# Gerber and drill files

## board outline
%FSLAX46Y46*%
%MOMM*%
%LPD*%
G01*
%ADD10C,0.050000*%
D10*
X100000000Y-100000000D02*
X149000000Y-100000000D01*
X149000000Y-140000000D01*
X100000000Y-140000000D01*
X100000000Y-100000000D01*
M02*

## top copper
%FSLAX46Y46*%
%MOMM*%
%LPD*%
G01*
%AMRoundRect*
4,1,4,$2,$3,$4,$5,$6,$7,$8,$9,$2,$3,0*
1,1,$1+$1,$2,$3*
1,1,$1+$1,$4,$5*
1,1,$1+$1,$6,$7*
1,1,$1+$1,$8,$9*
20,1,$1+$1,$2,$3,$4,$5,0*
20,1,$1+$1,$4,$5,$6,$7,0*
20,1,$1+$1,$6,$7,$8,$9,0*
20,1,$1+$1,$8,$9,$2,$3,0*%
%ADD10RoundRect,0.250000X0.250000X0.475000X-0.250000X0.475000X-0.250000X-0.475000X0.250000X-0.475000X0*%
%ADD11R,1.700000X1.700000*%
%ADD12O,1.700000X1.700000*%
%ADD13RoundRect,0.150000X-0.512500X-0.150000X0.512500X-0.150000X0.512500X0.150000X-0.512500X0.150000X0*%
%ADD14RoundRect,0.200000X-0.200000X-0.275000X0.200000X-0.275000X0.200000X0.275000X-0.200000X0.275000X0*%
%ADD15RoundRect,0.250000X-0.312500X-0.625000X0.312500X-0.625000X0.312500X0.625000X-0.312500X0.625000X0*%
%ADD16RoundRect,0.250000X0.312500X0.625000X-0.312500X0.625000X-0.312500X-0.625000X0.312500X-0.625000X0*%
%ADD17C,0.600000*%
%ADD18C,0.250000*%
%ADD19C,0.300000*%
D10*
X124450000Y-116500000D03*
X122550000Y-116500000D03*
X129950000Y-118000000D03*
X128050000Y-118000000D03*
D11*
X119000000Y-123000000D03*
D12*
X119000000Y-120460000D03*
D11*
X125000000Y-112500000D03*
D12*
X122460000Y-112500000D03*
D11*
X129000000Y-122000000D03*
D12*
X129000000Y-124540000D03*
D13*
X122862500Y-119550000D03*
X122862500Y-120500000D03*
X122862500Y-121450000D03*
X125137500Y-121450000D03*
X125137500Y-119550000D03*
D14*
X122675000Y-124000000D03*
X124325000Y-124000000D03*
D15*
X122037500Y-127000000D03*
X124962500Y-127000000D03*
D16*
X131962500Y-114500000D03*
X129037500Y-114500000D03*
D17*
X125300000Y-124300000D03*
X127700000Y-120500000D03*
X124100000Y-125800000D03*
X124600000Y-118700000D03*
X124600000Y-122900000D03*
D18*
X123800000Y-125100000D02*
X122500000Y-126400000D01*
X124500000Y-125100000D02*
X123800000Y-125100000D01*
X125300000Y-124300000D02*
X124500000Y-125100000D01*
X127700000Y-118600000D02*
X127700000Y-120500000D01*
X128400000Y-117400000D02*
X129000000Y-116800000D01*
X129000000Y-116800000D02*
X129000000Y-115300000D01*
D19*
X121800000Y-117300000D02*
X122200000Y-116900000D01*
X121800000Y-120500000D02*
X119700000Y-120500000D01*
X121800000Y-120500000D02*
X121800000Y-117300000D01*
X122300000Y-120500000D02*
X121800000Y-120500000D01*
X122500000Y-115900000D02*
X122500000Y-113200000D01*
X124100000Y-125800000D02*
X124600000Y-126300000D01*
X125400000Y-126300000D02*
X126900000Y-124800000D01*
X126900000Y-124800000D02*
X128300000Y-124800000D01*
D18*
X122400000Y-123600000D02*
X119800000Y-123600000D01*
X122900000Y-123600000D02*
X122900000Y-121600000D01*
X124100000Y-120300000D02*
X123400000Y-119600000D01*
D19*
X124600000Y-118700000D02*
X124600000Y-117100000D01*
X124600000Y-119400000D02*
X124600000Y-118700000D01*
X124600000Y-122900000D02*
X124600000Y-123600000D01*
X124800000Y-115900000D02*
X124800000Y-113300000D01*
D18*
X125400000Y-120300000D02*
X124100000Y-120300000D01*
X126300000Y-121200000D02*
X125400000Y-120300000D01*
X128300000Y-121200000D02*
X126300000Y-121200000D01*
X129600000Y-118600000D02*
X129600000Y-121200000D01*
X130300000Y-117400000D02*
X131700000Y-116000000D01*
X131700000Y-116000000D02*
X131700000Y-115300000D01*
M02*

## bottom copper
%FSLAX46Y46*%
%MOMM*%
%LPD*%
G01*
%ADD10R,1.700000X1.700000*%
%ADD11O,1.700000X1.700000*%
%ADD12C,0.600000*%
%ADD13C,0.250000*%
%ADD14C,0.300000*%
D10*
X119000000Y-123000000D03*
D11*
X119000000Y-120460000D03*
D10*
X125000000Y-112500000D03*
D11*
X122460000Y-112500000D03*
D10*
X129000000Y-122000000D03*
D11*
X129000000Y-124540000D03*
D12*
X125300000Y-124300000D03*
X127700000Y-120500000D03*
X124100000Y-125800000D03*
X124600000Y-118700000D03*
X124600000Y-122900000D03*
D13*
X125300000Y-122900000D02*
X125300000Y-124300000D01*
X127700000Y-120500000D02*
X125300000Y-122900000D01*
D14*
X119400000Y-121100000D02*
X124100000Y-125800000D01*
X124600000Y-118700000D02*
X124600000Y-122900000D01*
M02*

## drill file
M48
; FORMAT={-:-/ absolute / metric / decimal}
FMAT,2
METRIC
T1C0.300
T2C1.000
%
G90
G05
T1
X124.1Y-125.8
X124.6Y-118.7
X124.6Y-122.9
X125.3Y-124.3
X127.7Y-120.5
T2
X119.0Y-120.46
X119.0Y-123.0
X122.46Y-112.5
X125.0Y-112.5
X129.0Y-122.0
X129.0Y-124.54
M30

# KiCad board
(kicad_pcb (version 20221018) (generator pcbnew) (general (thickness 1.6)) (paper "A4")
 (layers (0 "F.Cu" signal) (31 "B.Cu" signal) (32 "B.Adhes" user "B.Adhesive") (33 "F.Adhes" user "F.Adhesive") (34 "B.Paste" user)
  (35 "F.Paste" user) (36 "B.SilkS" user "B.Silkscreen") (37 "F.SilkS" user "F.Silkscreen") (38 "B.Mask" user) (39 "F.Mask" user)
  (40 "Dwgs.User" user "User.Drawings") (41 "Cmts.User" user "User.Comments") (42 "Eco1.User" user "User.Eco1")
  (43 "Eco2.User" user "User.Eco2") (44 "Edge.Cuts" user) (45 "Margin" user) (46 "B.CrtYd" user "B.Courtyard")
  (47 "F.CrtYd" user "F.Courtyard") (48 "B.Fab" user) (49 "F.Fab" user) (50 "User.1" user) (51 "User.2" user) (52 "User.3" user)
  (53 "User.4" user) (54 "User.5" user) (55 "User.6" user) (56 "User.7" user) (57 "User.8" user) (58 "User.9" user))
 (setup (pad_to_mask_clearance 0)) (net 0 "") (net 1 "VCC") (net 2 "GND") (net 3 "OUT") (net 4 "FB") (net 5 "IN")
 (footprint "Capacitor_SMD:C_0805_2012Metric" (layer "F.Cu") (at 123.5 116.5 180)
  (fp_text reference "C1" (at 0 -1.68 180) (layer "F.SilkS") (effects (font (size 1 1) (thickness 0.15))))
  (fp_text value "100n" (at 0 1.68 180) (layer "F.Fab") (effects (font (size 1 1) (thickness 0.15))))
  (pad "1" smd roundrect (at -0.95 0 180) (size 1 1.45) (layers "F.Cu" "F.Paste" "F.Mask") (roundrect_rratio 0.25) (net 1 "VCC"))
  (pad "2" smd roundrect (at 0.95 0 180) (size 1 1.45) (layers "F.Cu" "F.Paste" "F.Mask") (roundrect_rratio 0.25) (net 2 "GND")))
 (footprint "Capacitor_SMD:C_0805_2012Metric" (layer "F.Cu") (at 129 118 180)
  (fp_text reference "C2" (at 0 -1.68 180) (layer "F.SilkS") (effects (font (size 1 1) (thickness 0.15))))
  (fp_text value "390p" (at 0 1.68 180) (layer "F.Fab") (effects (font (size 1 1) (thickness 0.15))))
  (pad "1" smd roundrect (at -0.95 0 180) (size 1 1.45) (layers "F.Cu" "F.Paste" "F.Mask") (roundrect_rratio 0.25) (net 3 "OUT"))
  (pad "2" smd roundrect (at 0.95 0 180) (size 1 1.45) (layers "F.Cu" "F.Paste" "F.Mask") (roundrect_rratio 0.25) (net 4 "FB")))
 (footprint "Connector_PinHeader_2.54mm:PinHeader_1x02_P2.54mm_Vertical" (layer "F.Cu") (at 119 123 180)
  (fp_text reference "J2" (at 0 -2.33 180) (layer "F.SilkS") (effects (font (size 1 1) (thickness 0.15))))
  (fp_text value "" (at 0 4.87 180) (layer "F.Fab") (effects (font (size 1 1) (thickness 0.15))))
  (pad "1" thru_hole rect (at 0 0 180) (size 1.7 1.7) (drill 1) (layers "*.Cu" "*.Mask") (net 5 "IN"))
  (pad "2" thru_hole oval (at 0 2.54 180) (size 1.7 1.7) (drill 1) (layers "*.Cu" "*.Mask") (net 2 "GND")))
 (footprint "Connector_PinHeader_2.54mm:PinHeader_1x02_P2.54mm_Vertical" (layer "F.Cu") (at 125 112.5 -90)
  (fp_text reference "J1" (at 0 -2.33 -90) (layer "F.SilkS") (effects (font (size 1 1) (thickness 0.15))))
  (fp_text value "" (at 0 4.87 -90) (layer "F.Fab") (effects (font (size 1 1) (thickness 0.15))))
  (pad "1" thru_hole rect (at 0 0 270) (size 1.7 1.7) (drill 1) (layers "*.Cu" "*.Mask") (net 1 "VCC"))
  (pad "2" thru_hole oval (at 0 2.54 270) (size 1.7 1.7) (drill 1) (layers "*.Cu" "*.Mask") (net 2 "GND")))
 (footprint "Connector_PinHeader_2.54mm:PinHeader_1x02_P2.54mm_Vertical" (layer "F.Cu") (at 129 122)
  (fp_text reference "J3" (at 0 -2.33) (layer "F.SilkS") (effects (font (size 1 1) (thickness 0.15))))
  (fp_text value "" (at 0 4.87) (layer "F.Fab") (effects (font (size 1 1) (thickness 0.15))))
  (pad "1" thru_hole rect (at 0 0) (size 1.7 1.7) (drill 1) (layers "*.Cu" "*.Mask") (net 3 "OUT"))
  (pad "2" thru_hole oval (at 0 2.54) (size 1.7 1.7) (drill 1) (layers "*.Cu" "*.Mask") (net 2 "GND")))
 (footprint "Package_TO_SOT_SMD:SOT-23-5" (layer "F.Cu") (at 124 120.5)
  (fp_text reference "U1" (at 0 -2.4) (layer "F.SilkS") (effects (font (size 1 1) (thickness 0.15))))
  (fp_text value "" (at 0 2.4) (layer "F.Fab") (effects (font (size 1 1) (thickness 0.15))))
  (pad "1" smd roundrect (at -1.1375 -0.95) (size 1.325 0.6) (layers "F.Cu" "F.Paste" "F.Mask") (roundrect_rratio 0.25) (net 3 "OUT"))
  (pad "2" smd roundrect (at -1.1375 0) (size 1.325 0.6) (layers "F.Cu" "F.Paste" "F.Mask") (roundrect_rratio 0.25) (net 2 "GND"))
  (pad "3" smd roundrect (at -1.1375 0.95) (size 1.325 0.6) (layers "F.Cu" "F.Paste" "F.Mask") (roundrect_rratio 0.25) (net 5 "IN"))
  (pad "4" smd roundrect (at 1.1375 0.95) (size 1.325 0.6) (layers "F.Cu" "F.Paste" "F.Mask") (roundrect_rratio 0.25))
  (pad "5" smd roundrect (at 1.1375 -0.95) (size 1.325 0.6) (layers "F.Cu" "F.Paste" "F.Mask") (roundrect_rratio 0.25) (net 1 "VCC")))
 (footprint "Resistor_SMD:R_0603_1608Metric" (layer "F.Cu") (at 123.5 124)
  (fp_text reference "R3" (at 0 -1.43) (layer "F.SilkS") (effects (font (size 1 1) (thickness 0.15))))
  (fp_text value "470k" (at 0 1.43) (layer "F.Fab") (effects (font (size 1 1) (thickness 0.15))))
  (pad "1" smd roundrect (at -0.825 0) (size 0.8 0.95) (layers "F.Cu" "F.Paste" "F.Mask") (roundrect_rratio 0.25) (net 5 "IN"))
  (pad "2" smd roundrect (at 0.825 0) (size 0.8 0.95) (layers "F.Cu" "F.Paste" "F.Mask") (roundrect_rratio 0.25) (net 1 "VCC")))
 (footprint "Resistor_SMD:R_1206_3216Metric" (layer "F.Cu") (at 123.5 127)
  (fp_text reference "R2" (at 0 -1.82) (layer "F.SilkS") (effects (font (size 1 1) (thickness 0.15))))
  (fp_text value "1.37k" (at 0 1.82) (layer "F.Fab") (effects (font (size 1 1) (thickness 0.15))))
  (pad "1" smd roundrect (at -1.4625 0) (size 1.125 1.75) (layers "F.Cu" "F.Paste" "F.Mask") (roundrect_rratio 0.222222) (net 4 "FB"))
  (pad "2" smd roundrect (at 1.4625 0) (size 1.125 1.75) (layers "F.Cu" "F.Paste" "F.Mask") (roundrect_rratio 0.222222) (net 2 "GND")))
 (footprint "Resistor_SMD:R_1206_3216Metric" (layer "F.Cu") (at 130.5 114.5 180)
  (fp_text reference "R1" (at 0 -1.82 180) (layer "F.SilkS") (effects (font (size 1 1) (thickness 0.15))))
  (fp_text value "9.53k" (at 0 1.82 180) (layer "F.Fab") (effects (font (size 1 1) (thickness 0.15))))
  (pad "1" smd roundrect (at -1.4625 0 180) (size 1.125 1.75) (layers "F.Cu" "F.Paste" "F.Mask") (roundrect_rratio 0.222222) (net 3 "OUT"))
  (pad "2" smd roundrect (at 1.4625 0 180) (size 1.125 1.75) (layers "F.Cu" "F.Paste" "F.Mask") (roundrect_rratio 0.222222) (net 4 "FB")))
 (gr_rect (start 100 100) (end 149 140) (stroke (width 0.05) (type default)) (fill none) (layer "Edge.Cuts"))
 (segment (start 123.8 125.1) (end 122.5 126.4) (width 0.25) (layer "F.Cu") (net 4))
 (segment (start 124.5 125.1) (end 123.8 125.1) (width 0.25) (layer "F.Cu") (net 4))
 (segment (start 125.3 124.3) (end 124.5 125.1) (width 0.25) (layer "F.Cu") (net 4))
 (segment (start 127.7 118.6) (end 127.7 120.5) (width 0.25) (layer "F.Cu") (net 4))
 (segment (start 128.4 117.4) (end 129 116.8) (width 0.25) (layer "F.Cu") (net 4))
 (segment (start 129 116.8) (end 129 115.3) (width 0.25) (layer "F.Cu") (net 4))
 (via (at 125.3 124.3) (size 0.6) (drill 0.3) (layers "F.Cu" "B.Cu") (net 4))
 (via (at 127.7 120.5) (size 0.6) (drill 0.3) (layers "F.Cu" "B.Cu") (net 4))
 (segment (start 121.8 117.3) (end 122.2 116.9) (width 0.3) (layer "F.Cu") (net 2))
 (segment (start 121.8 120.5) (end 119.7 120.5) (width 0.3) (layer "F.Cu") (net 2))
 (segment (start 121.8 120.5) (end 121.8 117.3) (width 0.3) (layer "F.Cu") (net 2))
 (segment (start 122.3 120.5) (end 121.8 120.5) (width 0.3) (layer "F.Cu") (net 2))
 (segment (start 122.5 115.9) (end 122.5 113.2) (width 0.3) (layer "F.Cu") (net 2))
 (segment (start 124.1 125.8) (end 124.6 126.3) (width 0.3) (layer "F.Cu") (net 2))
 (segment (start 125.3 122.9) (end 125.3 124.3) (width 0.25) (layer "B.Cu") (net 4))
 (segment (start 125.4 126.3) (end 126.9 124.8) (width 0.3) (layer "F.Cu") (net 2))
 (segment (start 126.9 124.8) (end 128.3 124.8) (width 0.3) (layer "F.Cu") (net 2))
 (segment (start 127.7 120.5) (end 125.3 122.9) (width 0.25) (layer "B.Cu") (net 4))
 (via (at 124.1 125.8) (size 0.6) (drill 0.3) (layers "F.Cu" "B.Cu") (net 2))
 (segment (start 119.4 121.1) (end 124.1 125.8) (width 0.3) (layer "B.Cu") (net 2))
 (segment (start 122.4 123.6) (end 119.8 123.6) (width 0.25) (layer "F.Cu") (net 5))
 (segment (start 122.9 123.6) (end 122.9 121.6) (width 0.25) (layer "F.Cu") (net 5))
 (segment (start 124.1 120.3) (end 123.4 119.6) (width 0.25) (layer "F.Cu") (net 3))
 (segment (start 124.6 118.7) (end 124.6 117.1) (width 0.3) (layer "F.Cu") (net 1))
 (segment (start 124.6 119.4) (end 124.6 118.7) (width 0.3) (layer "F.Cu") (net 1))
 (segment (start 124.6 122.9) (end 124.6 123.6) (width 0.3) (layer "F.Cu") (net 1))
 (segment (start 124.8 115.9) (end 124.8 113.3) (width 0.3) (layer "F.Cu") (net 1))
 (segment (start 125.4 120.3) (end 124.1 120.3) (width 0.25) (layer "F.Cu") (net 3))
 (segment (start 126.3 121.2) (end 125.4 120.3) (width 0.25) (layer "F.Cu") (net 3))
 (segment (start 128.3 121.2) (end 126.3 121.2) (width 0.25) (layer "F.Cu") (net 3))
 (segment (start 129.6 118.6) (end 129.6 121.2) (width 0.25) (layer "F.Cu") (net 3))
 (segment (start 130.3 117.4) (end 131.7 116) (width 0.25) (layer "F.Cu") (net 3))
 (segment (start 131.7 116) (end 131.7 115.3) (width 0.25) (layer "F.Cu") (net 3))
 (via (at 124.6 118.7) (size 0.6) (drill 0.3) (layers "F.Cu" "B.Cu") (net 1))
 (via (at 124.6 122.9) (size 0.6) (drill 0.3) (layers "F.Cu" "B.Cu") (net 1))
 (segment (start 124.6 118.7) (end 124.6 122.9) (width 0.3) (layer "B.Cu") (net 1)))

